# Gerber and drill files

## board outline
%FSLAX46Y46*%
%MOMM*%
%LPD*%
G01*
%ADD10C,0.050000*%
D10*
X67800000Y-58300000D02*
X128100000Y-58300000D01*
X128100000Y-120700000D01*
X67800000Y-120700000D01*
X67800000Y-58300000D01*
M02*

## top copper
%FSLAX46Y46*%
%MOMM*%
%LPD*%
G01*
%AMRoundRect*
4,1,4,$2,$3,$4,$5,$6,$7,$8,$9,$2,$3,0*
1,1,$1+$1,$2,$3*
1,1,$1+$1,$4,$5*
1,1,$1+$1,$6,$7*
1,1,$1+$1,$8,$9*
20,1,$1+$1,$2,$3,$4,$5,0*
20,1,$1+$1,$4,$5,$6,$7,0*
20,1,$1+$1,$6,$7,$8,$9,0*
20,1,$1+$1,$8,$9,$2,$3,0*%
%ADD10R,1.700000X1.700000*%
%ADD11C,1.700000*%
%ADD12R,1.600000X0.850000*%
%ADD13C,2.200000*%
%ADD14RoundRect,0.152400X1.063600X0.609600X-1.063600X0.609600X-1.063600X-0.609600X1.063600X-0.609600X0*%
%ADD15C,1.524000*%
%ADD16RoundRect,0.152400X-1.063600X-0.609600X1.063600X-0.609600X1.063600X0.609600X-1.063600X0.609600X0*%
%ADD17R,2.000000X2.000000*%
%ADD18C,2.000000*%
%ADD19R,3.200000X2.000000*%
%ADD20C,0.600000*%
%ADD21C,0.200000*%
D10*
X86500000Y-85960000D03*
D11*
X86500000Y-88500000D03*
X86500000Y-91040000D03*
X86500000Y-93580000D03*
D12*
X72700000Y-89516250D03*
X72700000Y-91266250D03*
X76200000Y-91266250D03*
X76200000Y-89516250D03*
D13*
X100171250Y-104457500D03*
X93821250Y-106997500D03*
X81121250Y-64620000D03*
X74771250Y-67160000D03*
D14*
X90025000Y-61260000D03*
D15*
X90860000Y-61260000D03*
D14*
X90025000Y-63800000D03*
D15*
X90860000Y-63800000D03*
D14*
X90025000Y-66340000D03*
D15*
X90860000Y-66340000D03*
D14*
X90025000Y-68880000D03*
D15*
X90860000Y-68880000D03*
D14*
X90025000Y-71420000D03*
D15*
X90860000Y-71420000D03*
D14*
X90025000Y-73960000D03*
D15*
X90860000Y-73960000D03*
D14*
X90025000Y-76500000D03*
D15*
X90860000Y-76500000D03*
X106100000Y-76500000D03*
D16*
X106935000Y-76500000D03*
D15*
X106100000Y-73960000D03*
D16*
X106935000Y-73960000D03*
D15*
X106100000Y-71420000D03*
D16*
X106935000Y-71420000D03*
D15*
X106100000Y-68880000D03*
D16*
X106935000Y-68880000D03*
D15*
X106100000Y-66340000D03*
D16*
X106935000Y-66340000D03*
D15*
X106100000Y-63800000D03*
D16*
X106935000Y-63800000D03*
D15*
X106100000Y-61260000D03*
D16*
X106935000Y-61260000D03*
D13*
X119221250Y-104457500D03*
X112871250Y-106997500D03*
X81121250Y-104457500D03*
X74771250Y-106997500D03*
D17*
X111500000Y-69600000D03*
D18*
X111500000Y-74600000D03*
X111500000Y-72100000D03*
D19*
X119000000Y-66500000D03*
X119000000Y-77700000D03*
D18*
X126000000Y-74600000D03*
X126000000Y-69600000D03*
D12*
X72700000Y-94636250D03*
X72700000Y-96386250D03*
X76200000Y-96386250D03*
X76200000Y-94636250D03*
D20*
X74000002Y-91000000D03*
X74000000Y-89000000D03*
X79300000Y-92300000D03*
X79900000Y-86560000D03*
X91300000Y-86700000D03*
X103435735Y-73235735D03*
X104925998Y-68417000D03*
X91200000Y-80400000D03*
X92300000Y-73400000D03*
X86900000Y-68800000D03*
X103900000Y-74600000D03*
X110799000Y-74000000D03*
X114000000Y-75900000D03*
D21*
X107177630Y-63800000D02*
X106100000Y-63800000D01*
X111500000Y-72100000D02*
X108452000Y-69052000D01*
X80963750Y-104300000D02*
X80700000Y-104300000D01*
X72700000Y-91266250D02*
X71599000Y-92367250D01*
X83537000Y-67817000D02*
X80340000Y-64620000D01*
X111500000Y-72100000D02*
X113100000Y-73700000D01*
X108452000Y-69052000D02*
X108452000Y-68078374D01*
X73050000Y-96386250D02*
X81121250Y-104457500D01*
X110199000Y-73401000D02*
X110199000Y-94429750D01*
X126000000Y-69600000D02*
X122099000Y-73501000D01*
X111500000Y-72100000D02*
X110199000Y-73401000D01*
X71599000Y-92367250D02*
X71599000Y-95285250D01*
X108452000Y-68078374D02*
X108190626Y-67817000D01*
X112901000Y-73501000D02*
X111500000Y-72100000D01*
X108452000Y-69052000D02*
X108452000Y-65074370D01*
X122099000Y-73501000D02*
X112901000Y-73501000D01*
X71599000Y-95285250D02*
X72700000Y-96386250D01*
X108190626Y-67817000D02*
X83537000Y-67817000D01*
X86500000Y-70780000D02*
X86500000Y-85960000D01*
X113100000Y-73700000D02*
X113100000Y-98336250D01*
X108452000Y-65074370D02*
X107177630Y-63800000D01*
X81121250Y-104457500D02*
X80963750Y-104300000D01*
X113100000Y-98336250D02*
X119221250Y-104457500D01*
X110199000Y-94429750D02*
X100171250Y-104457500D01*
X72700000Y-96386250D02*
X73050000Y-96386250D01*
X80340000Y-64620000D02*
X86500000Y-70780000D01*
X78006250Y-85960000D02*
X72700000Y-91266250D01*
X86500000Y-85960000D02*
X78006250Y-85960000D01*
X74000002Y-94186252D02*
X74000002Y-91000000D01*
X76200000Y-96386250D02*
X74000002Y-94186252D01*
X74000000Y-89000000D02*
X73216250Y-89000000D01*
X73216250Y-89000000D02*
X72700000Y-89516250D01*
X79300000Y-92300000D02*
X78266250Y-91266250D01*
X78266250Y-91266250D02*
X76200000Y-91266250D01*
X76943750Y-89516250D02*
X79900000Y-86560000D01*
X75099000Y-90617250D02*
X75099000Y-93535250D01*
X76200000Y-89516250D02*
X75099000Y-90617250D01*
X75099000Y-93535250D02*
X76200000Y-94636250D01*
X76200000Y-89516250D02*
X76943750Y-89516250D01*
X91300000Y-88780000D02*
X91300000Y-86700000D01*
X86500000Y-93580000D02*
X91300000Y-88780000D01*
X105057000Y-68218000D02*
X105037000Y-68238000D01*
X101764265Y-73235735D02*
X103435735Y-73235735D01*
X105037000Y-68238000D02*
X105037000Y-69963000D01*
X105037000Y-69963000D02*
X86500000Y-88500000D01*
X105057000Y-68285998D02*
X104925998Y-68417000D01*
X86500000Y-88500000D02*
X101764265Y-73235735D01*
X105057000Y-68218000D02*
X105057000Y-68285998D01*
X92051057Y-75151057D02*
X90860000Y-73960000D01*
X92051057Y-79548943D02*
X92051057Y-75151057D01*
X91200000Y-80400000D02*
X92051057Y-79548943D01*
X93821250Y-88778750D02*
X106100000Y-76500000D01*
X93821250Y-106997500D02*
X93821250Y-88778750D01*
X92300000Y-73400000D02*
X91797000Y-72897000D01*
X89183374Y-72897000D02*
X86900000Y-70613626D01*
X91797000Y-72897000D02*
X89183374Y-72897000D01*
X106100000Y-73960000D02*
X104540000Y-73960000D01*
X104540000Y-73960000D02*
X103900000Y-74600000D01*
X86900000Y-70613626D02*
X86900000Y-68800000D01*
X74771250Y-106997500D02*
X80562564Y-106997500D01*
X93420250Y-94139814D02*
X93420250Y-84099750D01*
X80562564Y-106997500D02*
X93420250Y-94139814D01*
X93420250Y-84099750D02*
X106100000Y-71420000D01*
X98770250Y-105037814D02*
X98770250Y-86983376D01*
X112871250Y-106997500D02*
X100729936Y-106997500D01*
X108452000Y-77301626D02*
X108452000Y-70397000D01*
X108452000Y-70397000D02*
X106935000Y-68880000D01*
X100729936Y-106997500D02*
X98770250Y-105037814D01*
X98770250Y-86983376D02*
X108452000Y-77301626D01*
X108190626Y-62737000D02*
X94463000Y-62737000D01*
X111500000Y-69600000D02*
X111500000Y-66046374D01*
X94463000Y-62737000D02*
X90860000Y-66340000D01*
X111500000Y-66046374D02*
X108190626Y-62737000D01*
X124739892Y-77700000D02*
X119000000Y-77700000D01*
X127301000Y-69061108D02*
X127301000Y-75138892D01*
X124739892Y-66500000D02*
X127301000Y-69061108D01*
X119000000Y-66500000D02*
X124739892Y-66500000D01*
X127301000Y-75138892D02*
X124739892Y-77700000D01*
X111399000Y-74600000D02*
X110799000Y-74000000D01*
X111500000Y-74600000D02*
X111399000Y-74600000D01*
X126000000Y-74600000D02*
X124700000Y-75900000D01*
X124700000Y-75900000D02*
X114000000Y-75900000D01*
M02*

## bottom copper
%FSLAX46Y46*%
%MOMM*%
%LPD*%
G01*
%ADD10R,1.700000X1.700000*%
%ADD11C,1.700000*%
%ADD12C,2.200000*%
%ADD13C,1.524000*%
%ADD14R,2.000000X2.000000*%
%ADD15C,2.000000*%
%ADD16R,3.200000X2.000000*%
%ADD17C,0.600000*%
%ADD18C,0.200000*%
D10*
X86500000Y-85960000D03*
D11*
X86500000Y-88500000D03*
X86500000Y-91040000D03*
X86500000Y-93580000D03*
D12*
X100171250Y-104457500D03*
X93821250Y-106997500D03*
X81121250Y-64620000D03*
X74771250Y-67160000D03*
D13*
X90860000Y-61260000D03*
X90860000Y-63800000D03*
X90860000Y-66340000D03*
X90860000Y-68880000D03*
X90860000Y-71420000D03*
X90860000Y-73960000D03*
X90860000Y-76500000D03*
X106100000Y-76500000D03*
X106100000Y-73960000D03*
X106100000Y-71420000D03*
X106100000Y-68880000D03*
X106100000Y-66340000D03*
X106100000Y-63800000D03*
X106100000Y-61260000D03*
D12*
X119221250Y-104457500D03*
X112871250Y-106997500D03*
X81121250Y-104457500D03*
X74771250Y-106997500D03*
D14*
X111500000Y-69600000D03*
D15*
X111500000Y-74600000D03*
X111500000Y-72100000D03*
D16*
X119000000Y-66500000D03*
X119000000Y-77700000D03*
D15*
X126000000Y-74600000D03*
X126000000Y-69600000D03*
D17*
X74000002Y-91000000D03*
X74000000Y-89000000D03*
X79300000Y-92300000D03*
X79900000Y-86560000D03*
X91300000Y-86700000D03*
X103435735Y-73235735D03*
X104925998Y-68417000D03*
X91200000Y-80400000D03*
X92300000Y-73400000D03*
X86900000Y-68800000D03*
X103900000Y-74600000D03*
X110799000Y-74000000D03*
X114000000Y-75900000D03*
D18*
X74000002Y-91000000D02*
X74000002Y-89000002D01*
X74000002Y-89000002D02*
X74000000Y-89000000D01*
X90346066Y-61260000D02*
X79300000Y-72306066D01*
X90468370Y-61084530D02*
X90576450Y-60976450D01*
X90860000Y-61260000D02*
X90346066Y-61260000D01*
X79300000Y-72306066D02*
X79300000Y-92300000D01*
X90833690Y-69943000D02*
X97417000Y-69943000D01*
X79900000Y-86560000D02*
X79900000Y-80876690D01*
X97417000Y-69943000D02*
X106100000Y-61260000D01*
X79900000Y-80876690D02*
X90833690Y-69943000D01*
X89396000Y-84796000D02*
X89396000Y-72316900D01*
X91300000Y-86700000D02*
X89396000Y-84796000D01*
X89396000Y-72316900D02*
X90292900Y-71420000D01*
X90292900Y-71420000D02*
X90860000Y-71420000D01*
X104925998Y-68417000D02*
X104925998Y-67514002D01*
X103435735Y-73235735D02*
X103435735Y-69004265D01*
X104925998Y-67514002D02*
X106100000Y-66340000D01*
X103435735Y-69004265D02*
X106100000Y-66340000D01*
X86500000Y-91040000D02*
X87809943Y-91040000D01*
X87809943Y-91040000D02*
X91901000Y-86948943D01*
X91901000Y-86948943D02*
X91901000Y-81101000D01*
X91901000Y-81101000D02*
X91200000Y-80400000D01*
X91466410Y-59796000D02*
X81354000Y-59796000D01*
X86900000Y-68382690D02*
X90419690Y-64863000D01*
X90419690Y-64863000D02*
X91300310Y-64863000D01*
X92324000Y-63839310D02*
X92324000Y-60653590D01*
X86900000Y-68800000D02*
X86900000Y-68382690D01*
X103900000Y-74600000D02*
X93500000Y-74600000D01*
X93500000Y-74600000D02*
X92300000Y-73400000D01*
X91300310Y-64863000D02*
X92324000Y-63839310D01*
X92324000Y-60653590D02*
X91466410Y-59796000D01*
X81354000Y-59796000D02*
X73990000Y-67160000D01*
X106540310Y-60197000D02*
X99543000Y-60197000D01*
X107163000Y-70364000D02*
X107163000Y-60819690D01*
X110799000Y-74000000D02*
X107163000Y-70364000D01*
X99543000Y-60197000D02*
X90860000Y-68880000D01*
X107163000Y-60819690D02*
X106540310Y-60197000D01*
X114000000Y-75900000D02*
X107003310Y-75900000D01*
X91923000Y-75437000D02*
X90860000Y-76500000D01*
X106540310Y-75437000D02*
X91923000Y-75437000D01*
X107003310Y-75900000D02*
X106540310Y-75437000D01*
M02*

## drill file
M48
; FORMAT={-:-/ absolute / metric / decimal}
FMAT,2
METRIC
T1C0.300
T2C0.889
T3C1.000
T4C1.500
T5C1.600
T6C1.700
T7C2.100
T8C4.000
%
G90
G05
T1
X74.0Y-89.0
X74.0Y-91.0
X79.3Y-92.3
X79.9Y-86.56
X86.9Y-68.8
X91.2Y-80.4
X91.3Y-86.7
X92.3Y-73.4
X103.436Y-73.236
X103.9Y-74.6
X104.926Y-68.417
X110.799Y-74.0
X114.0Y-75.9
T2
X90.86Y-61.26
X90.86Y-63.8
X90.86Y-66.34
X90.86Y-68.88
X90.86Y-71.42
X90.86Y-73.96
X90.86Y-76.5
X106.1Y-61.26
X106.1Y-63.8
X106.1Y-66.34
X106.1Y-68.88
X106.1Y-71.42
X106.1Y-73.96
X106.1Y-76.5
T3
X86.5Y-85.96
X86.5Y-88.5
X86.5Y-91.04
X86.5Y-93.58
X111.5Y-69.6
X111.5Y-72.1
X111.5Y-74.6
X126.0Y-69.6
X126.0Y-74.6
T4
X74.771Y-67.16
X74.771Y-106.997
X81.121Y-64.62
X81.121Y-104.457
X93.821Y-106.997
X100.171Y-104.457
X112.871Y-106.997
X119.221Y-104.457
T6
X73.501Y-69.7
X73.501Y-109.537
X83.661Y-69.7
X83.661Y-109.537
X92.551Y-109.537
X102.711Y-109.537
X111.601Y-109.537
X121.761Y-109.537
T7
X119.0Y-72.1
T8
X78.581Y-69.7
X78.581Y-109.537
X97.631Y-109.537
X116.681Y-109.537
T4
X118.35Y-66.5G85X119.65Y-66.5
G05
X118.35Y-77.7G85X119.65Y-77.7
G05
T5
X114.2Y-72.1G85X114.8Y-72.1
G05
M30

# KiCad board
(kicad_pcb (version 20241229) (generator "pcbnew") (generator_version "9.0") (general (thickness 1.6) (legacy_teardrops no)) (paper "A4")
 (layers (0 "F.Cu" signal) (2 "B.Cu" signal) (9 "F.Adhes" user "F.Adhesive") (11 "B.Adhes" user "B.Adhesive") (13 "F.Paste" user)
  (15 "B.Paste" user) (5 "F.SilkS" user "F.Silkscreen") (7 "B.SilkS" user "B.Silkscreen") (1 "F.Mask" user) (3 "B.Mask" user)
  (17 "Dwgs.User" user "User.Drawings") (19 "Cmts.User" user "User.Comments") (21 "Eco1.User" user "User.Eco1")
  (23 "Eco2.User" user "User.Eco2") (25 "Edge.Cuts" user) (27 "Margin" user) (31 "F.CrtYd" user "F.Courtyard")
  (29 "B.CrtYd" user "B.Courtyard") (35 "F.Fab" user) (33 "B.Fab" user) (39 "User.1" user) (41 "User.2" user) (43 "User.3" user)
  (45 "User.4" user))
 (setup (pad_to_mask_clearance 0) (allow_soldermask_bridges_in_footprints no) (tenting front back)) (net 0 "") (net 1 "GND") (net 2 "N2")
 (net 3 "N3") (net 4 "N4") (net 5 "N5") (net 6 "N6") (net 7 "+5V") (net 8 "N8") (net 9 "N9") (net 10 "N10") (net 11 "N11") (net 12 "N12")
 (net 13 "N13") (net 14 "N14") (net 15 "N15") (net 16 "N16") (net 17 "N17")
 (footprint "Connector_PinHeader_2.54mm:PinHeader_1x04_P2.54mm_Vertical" (layer "F.Cu") (at 86.5 85.96)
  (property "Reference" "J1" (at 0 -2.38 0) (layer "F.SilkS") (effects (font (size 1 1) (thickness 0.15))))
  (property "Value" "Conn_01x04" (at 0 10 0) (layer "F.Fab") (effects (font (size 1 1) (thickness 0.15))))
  (pad "1" thru_hole rect (at 0 0) (size 1.7 1.7) (drill 1) (layers "*.Cu" "*.Mask") (remove_unused_layers no) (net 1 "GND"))
  (pad "2" thru_hole circle (at 0 2.54) (size 1.7 1.7) (drill 1) (layers "*.Cu" "*.Mask") (remove_unused_layers no) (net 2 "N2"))
  (pad "3" thru_hole circle (at 0 5.08) (size 1.7 1.7) (drill 1) (layers "*.Cu" "*.Mask") (remove_unused_layers no) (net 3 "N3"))
  (pad "4" thru_hole circle (at 0 7.62) (size 1.7 1.7) (drill 1) (layers "*.Cu" "*.Mask") (remove_unused_layers no) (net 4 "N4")))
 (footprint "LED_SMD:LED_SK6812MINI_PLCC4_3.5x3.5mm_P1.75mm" (layer "F.Cu") (at 74.45 90.39125)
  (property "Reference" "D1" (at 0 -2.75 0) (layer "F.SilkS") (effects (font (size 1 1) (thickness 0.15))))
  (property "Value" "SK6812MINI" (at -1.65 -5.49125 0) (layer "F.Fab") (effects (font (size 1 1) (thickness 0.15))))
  (pad "1" smd rect (at -1.75 -0.875) (size 1.6 0.85) (layers "F.Cu" "F.Mask" "F.Paste") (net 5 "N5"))
  (pad "2" smd rect (at -1.75 0.875) (size 1.6 0.85) (layers "F.Cu" "F.Mask" "F.Paste") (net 1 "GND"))
  (pad "3" smd rect (at 1.75 0.875) (size 1.6 0.85) (layers "F.Cu" "F.Mask" "F.Paste") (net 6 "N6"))
  (pad "4" smd rect (at 1.75 -0.875) (size 1.6 0.85) (layers "F.Cu" "F.Mask" "F.Paste") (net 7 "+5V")))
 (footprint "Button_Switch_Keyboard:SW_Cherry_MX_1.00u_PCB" (layer "F.Cu") (at 100.17125 104.4575)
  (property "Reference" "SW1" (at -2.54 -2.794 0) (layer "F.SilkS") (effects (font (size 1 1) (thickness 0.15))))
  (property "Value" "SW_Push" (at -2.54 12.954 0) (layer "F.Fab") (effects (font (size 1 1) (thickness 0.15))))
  (pad "" np_thru_hole circle (at -7.62 5.08) (size 1.7 1.7) (drill 1.7) (layers "*.Cu" "*.Mask"))
  (pad "" np_thru_hole circle (at -2.54 5.08) (size 4 4) (drill 4) (layers "*.Cu" "*.Mask"))
  (pad "" np_thru_hole circle (at 2.54 5.08) (size 1.7 1.7) (drill 1.7) (layers "*.Cu" "*.Mask"))
  (pad "1" thru_hole circle (at 0 0) (size 2.2 2.2) (drill 1.5) (layers "*.Cu" "*.Mask") (remove_unused_layers no) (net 1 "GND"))
  (pad "2" thru_hole circle (at -6.35 2.54) (size 2.2 2.2) (drill 1.5) (layers "*.Cu" "*.Mask") (remove_unused_layers no) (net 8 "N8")))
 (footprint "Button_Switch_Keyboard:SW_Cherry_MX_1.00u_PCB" (layer "F.Cu") (at 81.12125 64.62)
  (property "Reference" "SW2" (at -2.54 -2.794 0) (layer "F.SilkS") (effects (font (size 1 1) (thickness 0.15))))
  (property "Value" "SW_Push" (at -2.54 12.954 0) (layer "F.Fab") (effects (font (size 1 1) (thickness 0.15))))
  (pad "" np_thru_hole circle (at -7.62 5.08) (size 1.7 1.7) (drill 1.7) (layers "*.Cu" "*.Mask"))
  (pad "" np_thru_hole circle (at -2.54 5.08) (size 4 4) (drill 4) (layers "*.Cu" "*.Mask"))
  (pad "" np_thru_hole circle (at 2.54 5.08) (size 1.7 1.7) (drill 1.7) (layers "*.Cu" "*.Mask"))
  (pad "1" thru_hole circle (at 0 0) (size 2.2 2.2) (drill 1.5) (layers "*.Cu" "*.Mask") (remove_unused_layers no) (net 1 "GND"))
  (pad "2" thru_hole circle (at -6.35 2.54) (size 2.2 2.2) (drill 1.5) (layers "*.Cu" "*.Mask") (remove_unused_layers no) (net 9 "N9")))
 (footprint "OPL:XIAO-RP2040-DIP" (layer "F.Cu") (at 98.48 68.88)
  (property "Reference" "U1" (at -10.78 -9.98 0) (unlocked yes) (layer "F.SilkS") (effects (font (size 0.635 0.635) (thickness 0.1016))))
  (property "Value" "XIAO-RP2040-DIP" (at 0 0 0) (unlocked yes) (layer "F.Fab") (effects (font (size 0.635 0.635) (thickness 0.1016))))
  (pad "1" smd roundrect (at -8.455 -7.62 180) (size 2.432 1.524) (layers "F.Cu" "F.Mask") (roundrect_rratio 0.1) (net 6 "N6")
   (thermal_bridge_angle 45))
  (pad "1" thru_hole circle (at -7.62 -7.62 180) (size 1.524 1.524) (drill 0.889) (layers "*.Cu" "*.Mask") (remove_unused_layers no)
   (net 6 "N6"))
  (pad "2" smd roundrect (at -8.455 -5.08 180) (size 2.432 1.524) (layers "F.Cu" "F.Mask") (roundrect_rratio 0.1) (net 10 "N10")
   (thermal_bridge_angle 45))
  (pad "2" thru_hole circle (at -7.62 -5.08 180) (size 1.524 1.524) (drill 0.889) (layers "*.Cu" "*.Mask") (remove_unused_layers no)
   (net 10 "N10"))
  (pad "3" smd roundrect (at -8.455 -2.54 180) (size 2.432 1.524) (layers "F.Cu" "F.Mask") (roundrect_rratio 0.1) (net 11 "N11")
   (thermal_bridge_angle 45))
  (pad "3" thru_hole circle (at -7.62 -2.54 180) (size 1.524 1.524) (drill 0.889) (layers "*.Cu" "*.Mask") (remove_unused_layers no)
   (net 11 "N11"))
  (pad "4" smd roundrect (at -8.455 0 180) (size 2.432 1.524) (layers "F.Cu" "F.Mask") (roundrect_rratio 0.1) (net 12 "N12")
   (thermal_bridge_angle 45))
  (pad "4" thru_hole circle (at -7.62 0 180) (size 1.524 1.524) (drill 0.889) (layers "*.Cu" "*.Mask") (remove_unused_layers no)
   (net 12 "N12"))
  (pad "5" smd roundrect (at -8.455 2.54 180) (size 2.432 1.524) (layers "F.Cu" "F.Mask") (roundrect_rratio 0.1) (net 4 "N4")
   (thermal_bridge_angle 45))
  (pad "5" thru_hole circle (at -7.62 2.54 180) (size 1.524 1.524) (drill 0.889) (layers "*.Cu" "*.Mask") (remove_unused_layers no)
   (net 4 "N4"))
  (pad "6" smd roundrect (at -8.455 5.08 180) (size 2.432 1.524) (layers "F.Cu" "F.Mask") (roundrect_rratio 0.1) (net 3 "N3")
   (thermal_bridge_angle 45))
  (pad "6" thru_hole circle (at -7.62 5.08 180) (size 1.524 1.524) (drill 0.889) (layers "*.Cu" "*.Mask") (remove_unused_layers no)
   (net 3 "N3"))
  (pad "7" smd roundrect (at -8.455 7.62 180) (size 2.432 1.524) (layers "F.Cu" "F.Mask") (roundrect_rratio 0.1) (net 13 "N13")
   (thermal_bridge_angle 45))
  (pad "7" thru_hole circle (at -7.62 7.62 180) (size 1.524 1.524) (drill 0.889) (layers "*.Cu" "*.Mask") (remove_unused_layers no)
   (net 13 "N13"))
  (pad "8" thru_hole circle (at 7.62 7.62) (size 1.524 1.524) (drill 0.889) (layers "*.Cu" "*.Mask") (remove_unused_layers no) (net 8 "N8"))
  (pad "8" smd roundrect (at 8.455 7.62) (size 2.432 1.524) (layers "F.Cu" "F.Mask") (roundrect_rratio 0.1) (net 8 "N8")
   (thermal_bridge_angle 45))
  (pad "9" thru_hole circle (at 7.62 5.08) (size 1.524 1.524) (drill 0.889) (layers "*.Cu" "*.Mask") (remove_unused_layers no) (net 9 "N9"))
  (pad "9" smd roundrect (at 8.455 5.08) (size 2.432 1.524) (layers "F.Cu" "F.Mask") (roundrect_rratio 0.1) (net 9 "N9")
   (thermal_bridge_angle 45))
  (pad "10" thru_hole circle (at 7.62 2.54) (size 1.524 1.524) (drill 0.889) (layers "*.Cu" "*.Mask") (remove_unused_layers no)
   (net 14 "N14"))
  (pad "10" smd roundrect (at 8.455 2.54) (size 2.432 1.524) (layers "F.Cu" "F.Mask") (roundrect_rratio 0.1) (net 14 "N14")
   (thermal_bridge_angle 45))
  (pad "11" thru_hole circle (at 7.62 0) (size 1.524 1.524) (drill 0.889) (layers "*.Cu" "*.Mask") (remove_unused_layers no) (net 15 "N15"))
  (pad "11" smd roundrect (at 8.455 0) (size 2.432 1.524) (layers "F.Cu" "F.Mask") (roundrect_rratio 0.1) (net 15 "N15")
   (thermal_bridge_angle 45))
  (pad "12" thru_hole circle (at 7.62 -2.54) (size 1.524 1.524) (drill 0.889) (layers "*.Cu" "*.Mask") (remove_unused_layers no)
   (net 2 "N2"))
  (pad "12" smd roundrect (at 8.455 -2.54) (size 2.432 1.524) (layers "F.Cu" "F.Mask") (roundrect_rratio 0.1) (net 2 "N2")
   (thermal_bridge_angle 45))
  (pad "13" thru_hole circle (at 7.62 -5.08) (size 1.524 1.524) (drill 0.889) (layers "*.Cu" "*.Mask") (remove_unused_layers no)
   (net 1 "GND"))
  (pad "13" smd roundrect (at 8.455 -5.08) (size 2.432 1.524) (layers "F.Cu" "F.Mask") (roundrect_rratio 0.1) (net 1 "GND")
   (thermal_bridge_angle 45))
  (pad "14" thru_hole circle (at 7.62 -7.62) (size 1.524 1.524) (drill 0.889) (layers "*.Cu" "*.Mask") (remove_unused_layers no)
   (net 7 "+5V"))
  (pad "14" smd roundrect (at 8.455 -7.62) (size 2.432 1.524) (layers "F.Cu" "F.Mask") (roundrect_rratio 0.1) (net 7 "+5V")
   (thermal_bridge_angle 45)))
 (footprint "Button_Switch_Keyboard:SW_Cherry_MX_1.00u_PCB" (layer "F.Cu") (at 119.22125 104.4575)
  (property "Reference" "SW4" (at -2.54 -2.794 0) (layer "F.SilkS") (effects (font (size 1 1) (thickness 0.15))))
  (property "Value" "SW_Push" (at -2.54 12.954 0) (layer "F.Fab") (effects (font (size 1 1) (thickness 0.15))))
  (pad "" np_thru_hole circle (at -7.62 5.08) (size 1.7 1.7) (drill 1.7) (layers "*.Cu" "*.Mask"))
  (pad "" np_thru_hole circle (at -2.54 5.08) (size 4 4) (drill 4) (layers "*.Cu" "*.Mask"))
  (pad "" np_thru_hole circle (at 2.54 5.08) (size 1.7 1.7) (drill 1.7) (layers "*.Cu" "*.Mask"))
  (pad "1" thru_hole circle (at 0 0) (size 2.2 2.2) (drill 1.5) (layers "*.Cu" "*.Mask") (remove_unused_layers no) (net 1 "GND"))
  (pad "2" thru_hole circle (at -6.35 2.54) (size 2.2 2.2) (drill 1.5) (layers "*.Cu" "*.Mask") (remove_unused_layers no) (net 15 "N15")))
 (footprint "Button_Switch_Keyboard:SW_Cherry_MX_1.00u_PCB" (layer "F.Cu") (at 81.12125 104.4575)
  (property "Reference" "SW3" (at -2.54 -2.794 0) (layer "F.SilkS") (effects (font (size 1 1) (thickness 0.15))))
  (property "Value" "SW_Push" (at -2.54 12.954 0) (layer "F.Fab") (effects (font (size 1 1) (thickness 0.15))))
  (pad "" np_thru_hole circle (at -7.62 5.08) (size 1.7 1.7) (drill 1.7) (layers "*.Cu" "*.Mask"))
  (pad "" np_thru_hole circle (at -2.54 5.08) (size 4 4) (drill 4) (layers "*.Cu" "*.Mask"))
  (pad "" np_thru_hole circle (at 2.54 5.08) (size 1.7 1.7) (drill 1.7) (layers "*.Cu" "*.Mask"))
  (pad "1" thru_hole circle (at 0 0) (size 2.2 2.2) (drill 1.5) (layers "*.Cu" "*.Mask") (remove_unused_layers no) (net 1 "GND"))
  (pad "2" thru_hole circle (at -6.35 2.54) (size 2.2 2.2) (drill 1.5) (layers "*.Cu" "*.Mask") (remove_unused_layers no) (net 14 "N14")))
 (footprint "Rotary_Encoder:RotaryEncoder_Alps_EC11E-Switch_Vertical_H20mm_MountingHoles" (layer "F.Cu") (at 111.5 69.6)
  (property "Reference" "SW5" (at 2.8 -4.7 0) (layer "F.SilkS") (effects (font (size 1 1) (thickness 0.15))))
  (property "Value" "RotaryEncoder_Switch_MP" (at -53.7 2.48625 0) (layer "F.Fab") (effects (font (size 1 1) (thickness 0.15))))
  (pad "" np_thru_hole oval (at 3 2.5) (size 2.2 1.6) (drill oval 2.2 1.6) (layers "*.Mask"))
  (pad "" np_thru_hole circle (at 7.5 2.5) (size 2.1 2.1) (drill 2.1) (layers "*.Mask"))
  (pad "A" thru_hole rect (at 0 0) (size 2 2) (drill 1) (layers "*.Cu" "*.Mask") (remove_unused_layers no) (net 11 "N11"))
  (pad "B" thru_hole circle (at 0 5) (size 2 2) (drill 1) (layers "*.Cu" "*.Mask") (remove_unused_layers no) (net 12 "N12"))
  (pad "C" thru_hole circle (at 0 2.5) (size 2 2) (drill 1) (layers "*.Cu" "*.Mask") (remove_unused_layers no) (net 1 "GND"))
  (pad "MP" thru_hole rect (at 7.5 -3.1) (size 3.2 2) (drill oval 2.8 1.5) (layers "*.Cu" "*.Mask") (remove_unused_layers no) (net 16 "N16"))
  (pad "MP" thru_hole rect (at 7.5 8.1) (size 3.2 2) (drill oval 2.8 1.5) (layers "*.Cu" "*.Mask") (remove_unused_layers no) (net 16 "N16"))
  (pad "S1" thru_hole circle (at 14.5 5) (size 2 2) (drill 1) (layers "*.Cu" "*.Mask") (remove_unused_layers no) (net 13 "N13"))
  (pad "S2" thru_hole circle (at 14.5 0) (size 2 2) (drill 1) (layers "*.Cu" "*.Mask") (remove_unused_layers no) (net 1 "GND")))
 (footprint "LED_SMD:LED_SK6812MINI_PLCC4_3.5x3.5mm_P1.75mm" (layer "F.Cu") (at 74.45 95.51125)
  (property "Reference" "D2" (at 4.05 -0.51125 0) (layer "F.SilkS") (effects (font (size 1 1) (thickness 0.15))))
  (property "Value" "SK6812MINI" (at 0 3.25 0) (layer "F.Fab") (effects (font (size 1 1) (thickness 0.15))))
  (pad "1" smd rect (at -1.75 -0.875) (size 1.6 0.85) (layers "F.Cu" "F.Mask" "F.Paste") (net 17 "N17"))
  (pad "2" smd rect (at -1.75 0.875) (size 1.6 0.85) (layers "F.Cu" "F.Mask" "F.Paste") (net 1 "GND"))
  (pad "3" smd rect (at 1.75 0.875) (size 1.6 0.85) (layers "F.Cu" "F.Mask" "F.Paste") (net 5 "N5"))
  (pad "4" smd rect (at 1.75 -0.875) (size 1.6 0.85) (layers "F.Cu" "F.Mask" "F.Paste") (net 7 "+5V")))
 (gr_rect (start 67.8 58.3) (end 128.1 120.7) (stroke (width 0.05) (type default)) (fill no) (layer "Edge.Cuts"))
 (segment (start 107.17763 63.8) (end 106.1 63.8) (width 0.2) (layer "F.Cu") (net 1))
 (segment (start 111.5 72.1) (end 108.452 69.052) (width 0.2) (layer "F.Cu") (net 1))
 (segment (start 80.96375 104.3) (end 80.7 104.3) (width 0.2) (layer "F.Cu") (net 1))
 (segment (start 72.7 91.26625) (end 71.599 92.36725) (width 0.2) (layer "F.Cu") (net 1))
 (segment (start 83.537 67.817) (end 80.34 64.62) (width 0.2) (layer "F.Cu") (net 1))
 (segment (start 111.5 72.1) (end 113.1 73.7) (width 0.2) (layer "F.Cu") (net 1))
 (segment (start 108.452 69.052) (end 108.452 68.078374) (width 0.2) (layer "F.Cu") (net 1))
 (segment (start 73.05 96.38625) (end 81.12125 104.4575) (width 0.2) (layer "F.Cu") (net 1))
 (segment (start 110.199 73.401) (end 110.199 94.42975) (width 0.2) (layer "F.Cu") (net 1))
 (segment (start 126 69.6) (end 122.099 73.501) (width 0.2) (layer "F.Cu") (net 1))
 (segment (start 111.5 72.1) (end 110.199 73.401) (width 0.2) (layer "F.Cu") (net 1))
 (segment (start 71.599 92.36725) (end 71.599 95.28525) (width 0.2) (layer "F.Cu") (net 1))
 (segment (start 108.452 68.078374) (end 108.190626 67.817) (width 0.2) (layer "F.Cu") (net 1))
 (segment (start 112.901 73.501) (end 111.5 72.1) (width 0.2) (layer "F.Cu") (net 1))
 (segment (start 108.452 69.052) (end 108.452 65.07437) (width 0.2) (layer "F.Cu") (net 1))
 (segment (start 122.099 73.501) (end 112.901 73.501) (width 0.2) (layer "F.Cu") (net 1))
 (segment (start 71.599 95.28525) (end 72.7 96.38625) (width 0.2) (layer "F.Cu") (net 1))
 (segment (start 108.190626 67.817) (end 83.537 67.817) (width 0.2) (layer "F.Cu") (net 1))
 (segment (start 86.5 70.78) (end 86.5 85.96) (width 0.2) (layer "F.Cu") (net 1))
 (segment (start 113.1 73.7) (end 113.1 98.33625) (width 0.2) (layer "F.Cu") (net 1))
 (segment (start 108.452 65.07437) (end 107.17763 63.8) (width 0.2) (layer "F.Cu") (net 1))
 (segment (start 81.12125 104.4575) (end 80.96375 104.3) (width 0.2) (layer "F.Cu") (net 1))
 (segment (start 113.1 98.33625) (end 119.22125 104.4575) (width 0.2) (layer "F.Cu") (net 1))
 (segment (start 110.199 94.42975) (end 100.17125 104.4575) (width 0.2) (layer "F.Cu") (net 1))
 (segment (start 72.7 96.38625) (end 73.05 96.38625) (width 0.2) (layer "F.Cu") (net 1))
 (segment (start 80.34 64.62) (end 86.5 70.78) (width 0.2) (layer "F.Cu") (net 1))
 (segment (start 78.00625 85.96) (end 72.7 91.26625) (width 0.2) (layer "F.Cu") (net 1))
 (segment (start 86.5 85.96) (end 78.00625 85.96) (width 0.2) (layer "F.Cu") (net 1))
 (segment (start 74.000002 94.186252) (end 74.000002 91) (width 0.2) (layer "F.Cu") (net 5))
 (segment (start 76.2 96.38625) (end 74.000002 94.186252) (width 0.2) (layer "F.Cu") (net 5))
 (segment (start 74 89) (end 73.21625 89) (width 0.2) (layer "F.Cu") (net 5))
 (segment (start 73.21625 89) (end 72.7 89.51625) (width 0.2) (layer "F.Cu") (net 5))
 (via (at 74.000002 91) (size 0.6) (drill 0.3) (layers "F.Cu" "B.Cu") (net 5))
 (via (at 74 89) (size 0.6) (drill 0.3) (layers "F.Cu" "B.Cu") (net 5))
 (segment (start 74.000002 91) (end 74.000002 89.000002) (width 0.2) (layer "B.Cu") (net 5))
 (segment (start 74.000002 89.000002) (end 74 89) (width 0.2) (layer "B.Cu") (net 5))
 (segment (start 79.3 92.3) (end 78.26625 91.26625) (width 0.2) (layer "F.Cu") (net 6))
 (segment (start 78.26625 91.26625) (end 76.2 91.26625) (width 0.2) (layer "F.Cu") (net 6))
 (via (at 79.3 92.3) (size 0.6) (drill 0.3) (layers "F.Cu" "B.Cu") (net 6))
 (segment (start 90.346066 61.26) (end 79.3 72.306066) (width 0.2) (layer "B.Cu") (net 6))
 (segment (start 90.46837 61.08453) (end 90.57645 60.97645) (width 0.2) (layer "B.Cu") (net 6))
 (segment (start 90.86 61.26) (end 90.346066 61.26) (width 0.2) (layer "B.Cu") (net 6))
 (segment (start 79.3 72.306066) (end 79.3 92.3) (width 0.2) (layer "B.Cu") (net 6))
 (segment (start 76.94375 89.51625) (end 79.9 86.56) (width 0.2) (layer "F.Cu") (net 7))
 (segment (start 75.099 90.61725) (end 75.099 93.53525) (width 0.2) (layer "F.Cu") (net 7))
 (segment (start 76.2 89.51625) (end 75.099 90.61725) (width 0.2) (layer "F.Cu") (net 7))
 (segment (start 75.099 93.53525) (end 76.2 94.63625) (width 0.2) (layer "F.Cu") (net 7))
 (segment (start 76.2 89.51625) (end 76.94375 89.51625) (width 0.2) (layer "F.Cu") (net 7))
 (via (at 79.9 86.56) (size 0.6) (drill 0.3) (layers "F.Cu" "B.Cu") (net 7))
 (segment (start 90.83369 69.943) (end 97.417 69.943) (width 0.2) (layer "B.Cu") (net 7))
 (segment (start 79.9 86.56) (end 79.9 80.87669) (width 0.2) (layer "B.Cu") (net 7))
 (segment (start 97.417 69.943) (end 106.1 61.26) (width 0.2) (layer "B.Cu") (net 7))
 (segment (start 79.9 80.87669) (end 90.83369 69.943) (width 0.2) (layer "B.Cu") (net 7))
 (segment (start 91.3 88.78) (end 91.3 86.7) (width 0.2) (layer "F.Cu") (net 4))
 (segment (start 86.5 93.58) (end 91.3 88.78) (width 0.2) (layer "F.Cu") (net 4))
 (via (at 91.3 86.7) (size 0.6) (drill 0.3) (layers "F.Cu" "B.Cu") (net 4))
 (segment (start 89.396 84.796) (end 89.396 72.3169) (width 0.2) (layer "B.Cu") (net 4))
 (segment (start 91.3 86.7) (end 89.396 84.796) (width 0.2) (layer "B.Cu") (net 4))
 (segment (start 89.396 72.3169) (end 90.2929 71.42) (width 0.2) (layer "B.Cu") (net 4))
 (segment (start 90.2929 71.42) (end 90.86 71.42) (width 0.2) (layer "B.Cu") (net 4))
 (segment (start 105.057 68.218) (end 105.037 68.238) (width 0.2) (layer "F.Cu") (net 2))
 (segment (start 101.764265 73.235735) (end 103.435735 73.235735) (width 0.2) (layer "F.Cu") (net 2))
 (segment (start 105.037 68.238) (end 105.037 69.963) (width 0.2) (layer "F.Cu") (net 2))
 (segment (start 105.037 69.963) (end 86.5 88.5) (width 0.2) (layer "F.Cu") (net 2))
 (segment (start 105.057 68.285998) (end 104.925998 68.417) (width 0.2) (layer "F.Cu") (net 2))
 (segment (start 86.5 88.5) (end 101.764265 73.235735) (width 0.2) (layer "F.Cu") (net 2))
 (segment (start 105.057 68.218) (end 105.057 68.285998) (width 0.2) (layer "F.Cu") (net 2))
 (via (at 103.435735 73.235735) (size 0.6) (drill 0.3) (layers "F.Cu" "B.Cu") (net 2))
 (via (at 104.925998 68.417) (size 0.6) (drill 0.3) (layers "F.Cu" "B.Cu") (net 2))
 (segment (start 104.925998 68.417) (end 104.925998 67.514002) (width 0.2) (layer "B.Cu") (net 2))
 (segment (start 103.435735 73.235735) (end 103.435735 69.004265) (width 0.2) (layer "B.Cu") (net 2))
 (segment (start 104.925998 67.514002) (end 106.1 66.34) (width 0.2) (layer "B.Cu") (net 2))
 (segment (start 103.435735 69.004265) (end 106.1 66.34) (width 0.2) (layer "B.Cu") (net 2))
 (segment (start 92.051057 75.151057) (end 90.86 73.96) (width 0.2) (layer "F.Cu") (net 3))
 (segment (start 92.051057 79.548943) (end 92.051057 75.151057) (width 0.2) (layer "F.Cu") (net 3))
 (segment (start 91.2 80.4) (end 92.051057 79.548943) (width 0.2) (layer "F.Cu") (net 3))
 (via (at 91.2 80.4) (size 0.6) (drill 0.3) (layers "F.Cu" "B.Cu") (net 3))
 (segment (start 86.5 91.04) (end 87.809943 91.04) (width 0.2) (layer "B.Cu") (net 3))
 (segment (start 87.809943 91.04) (end 91.901 86.948943) (width 0.2) (layer "B.Cu") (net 3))
 (segment (start 91.901 86.948943) (end 91.901 81.101) (width 0.2) (layer "B.Cu") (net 3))
 (segment (start 91.901 81.101) (end 91.2 80.4) (width 0.2) (layer "B.Cu") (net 3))
 (segment (start 93.82125 88.77875) (end 106.1 76.5) (width 0.2) (layer "F.Cu") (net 8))
 (segment (start 93.82125 106.9975) (end 93.82125 88.77875) (width 0.2) (layer "F.Cu") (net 8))
 (segment (start 92.3 73.4) (end 91.797 72.897) (width 0.2) (layer "F.Cu") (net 9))
 (segment (start 89.183374 72.897) (end 86.9 70.613626) (width 0.2) (layer "F.Cu") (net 9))
 (segment (start 91.797 72.897) (end 89.183374 72.897) (width 0.2) (layer "F.Cu") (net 9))
 (segment (start 106.1 73.96) (end 104.54 73.96) (width 0.2) (layer "F.Cu") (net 9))
 (segment (start 104.54 73.96) (end 103.9 74.6) (width 0.2) (layer "F.Cu") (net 9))
 (segment (start 86.9 70.613626) (end 86.9 68.8) (width 0.2) (layer "F.Cu") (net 9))
 (via (at 92.3 73.4) (size 0.6) (drill 0.3) (layers "F.Cu" "B.Cu") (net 9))
 (via (at 86.9 68.8) (size 0.6) (drill 0.3) (layers "F.Cu" "B.Cu") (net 9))
 (via (at 103.9 74.6) (size 0.6) (drill 0.3) (layers "F.Cu" "B.Cu") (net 9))
 (segment (start 91.46641 59.796) (end 81.354 59.796) (width 0.2) (layer "B.Cu") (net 9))
 (segment (start 86.9 68.38269) (end 90.41969 64.863) (width 0.2) (layer "B.Cu") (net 9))
 (segment (start 90.41969 64.863) (end 91.30031 64.863) (width 0.2) (layer "B.Cu") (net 9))
 (segment (start 92.324 63.83931) (end 92.324 60.65359) (width 0.2) (layer "B.Cu") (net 9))
 (segment (start 86.9 68.8) (end 86.9 68.38269) (width 0.2) (layer "B.Cu") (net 9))
 (segment (start 103.9 74.6) (end 93.5 74.6) (width 0.2) (layer "B.Cu") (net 9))
 (segment (start 93.5 74.6) (end 92.3 73.4) (width 0.2) (layer "B.Cu") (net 9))
 (segment (start 91.30031 64.863) (end 92.324 63.83931) (width 0.2) (layer "B.Cu") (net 9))
 (segment (start 92.324 60.65359) (end 91.46641 59.796) (width 0.2) (layer "B.Cu") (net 9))
 (segment (start 81.354 59.796) (end 73.99 67.16) (width 0.2) (layer "B.Cu") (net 9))
 (segment (start 74.77125 106.9975) (end 80.562564 106.9975) (width 0.2) (layer "F.Cu") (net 14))
 (segment (start 93.42025 94.139814) (end 93.42025 84.09975) (width 0.2) (layer "F.Cu") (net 14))
 (segment (start 80.562564 106.9975) (end 93.42025 94.139814) (width 0.2) (layer "F.Cu") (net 14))
 (segment (start 93.42025 84.09975) (end 106.1 71.42) (width 0.2) (layer "F.Cu") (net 14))
 (segment (start 98.77025 105.037814) (end 98.77025 86.983376) (width 0.2) (layer "F.Cu") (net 15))
 (segment (start 112.87125 106.9975) (end 100.729936 106.9975) (width 0.2) (layer "F.Cu") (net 15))
 (segment (start 108.452 77.301626) (end 108.452 70.397) (width 0.2) (layer "F.Cu") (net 15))
 (segment (start 108.452 70.397) (end 106.935 68.88) (width 0.2) (layer "F.Cu") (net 15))
 (segment (start 100.729936 106.9975) (end 98.77025 105.037814) (width 0.2) (layer "F.Cu") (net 15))
 (segment (start 98.77025 86.983376) (end 108.452 77.301626) (width 0.2) (layer "F.Cu") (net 15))
 (segment (start 108.190626 62.737) (end 94.463 62.737) (width 0.2) (layer "F.Cu") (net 11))
 (segment (start 111.5 69.6) (end 111.5 66.046374) (width 0.2) (layer "F.Cu") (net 11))
 (segment (start 94.463 62.737) (end 90.86 66.34) (width 0.2) (layer "F.Cu") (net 11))
 (segment (start 111.5 66.046374) (end 108.190626 62.737) (width 0.2) (layer "F.Cu") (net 11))
 (segment (start 124.739892 77.7) (end 119 77.7) (width 0.2) (layer "F.Cu") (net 16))
 (segment (start 127.301 69.061108) (end 127.301 75.138892) (width 0.2) (layer "F.Cu") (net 16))
 (segment (start 124.739892 66.5) (end 127.301 69.061108) (width 0.2) (layer "F.Cu") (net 16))
 (segment (start 119 66.5) (end 124.739892 66.5) (width 0.2) (layer "F.Cu") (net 16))
 (segment (start 127.301 75.138892) (end 124.739892 77.7) (width 0.2) (layer "F.Cu") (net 16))
 (segment (start 111.399 74.6) (end 110.799 74) (width 0.2) (layer "F.Cu") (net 12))
 (segment (start 111.5 74.6) (end 111.399 74.6) (width 0.2) (layer "F.Cu") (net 12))
 (via (at 110.799 74) (size 0.6) (drill 0.3) (layers "F.Cu" "B.Cu") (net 12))
 (segment (start 106.54031 60.197) (end 99.543 60.197) (width 0.2) (layer "B.Cu") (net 12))
 (segment (start 107.163 70.364) (end 107.163 60.81969) (width 0.2) (layer "B.Cu") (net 12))
 (segment (start 110.799 74) (end 107.163 70.364) (width 0.2) (layer "B.Cu") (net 12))
 (segment (start 99.543 60.197) (end 90.86 68.88) (width 0.2) (layer "B.Cu") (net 12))
 (segment (start 107.163 60.81969) (end 106.54031 60.197) (width 0.2) (layer "B.Cu") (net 12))
 (segment (start 126 74.6) (end 124.7 75.9) (width 0.2) (layer "F.Cu") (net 13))
 (segment (start 124.7 75.9) (end 114 75.9) (width 0.2) (layer "F.Cu") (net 13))
 (via (at 114 75.9) (size 0.6) (drill 0.3) (layers "F.Cu" "B.Cu") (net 13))
 (segment (start 114 75.9) (end 107.00331 75.9) (width 0.2) (layer "B.Cu") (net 13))
 (segment (start 91.923 75.437) (end 90.86 76.5) (width 0.2) (layer "B.Cu") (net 13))
 (segment (start 106.54031 75.437) (end 91.923 75.437) (width 0.2) (layer "B.Cu") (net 13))
 (segment (start 107.00331 75.9) (end 106.54031 75.437) (width 0.2) (layer "B.Cu") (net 13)))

